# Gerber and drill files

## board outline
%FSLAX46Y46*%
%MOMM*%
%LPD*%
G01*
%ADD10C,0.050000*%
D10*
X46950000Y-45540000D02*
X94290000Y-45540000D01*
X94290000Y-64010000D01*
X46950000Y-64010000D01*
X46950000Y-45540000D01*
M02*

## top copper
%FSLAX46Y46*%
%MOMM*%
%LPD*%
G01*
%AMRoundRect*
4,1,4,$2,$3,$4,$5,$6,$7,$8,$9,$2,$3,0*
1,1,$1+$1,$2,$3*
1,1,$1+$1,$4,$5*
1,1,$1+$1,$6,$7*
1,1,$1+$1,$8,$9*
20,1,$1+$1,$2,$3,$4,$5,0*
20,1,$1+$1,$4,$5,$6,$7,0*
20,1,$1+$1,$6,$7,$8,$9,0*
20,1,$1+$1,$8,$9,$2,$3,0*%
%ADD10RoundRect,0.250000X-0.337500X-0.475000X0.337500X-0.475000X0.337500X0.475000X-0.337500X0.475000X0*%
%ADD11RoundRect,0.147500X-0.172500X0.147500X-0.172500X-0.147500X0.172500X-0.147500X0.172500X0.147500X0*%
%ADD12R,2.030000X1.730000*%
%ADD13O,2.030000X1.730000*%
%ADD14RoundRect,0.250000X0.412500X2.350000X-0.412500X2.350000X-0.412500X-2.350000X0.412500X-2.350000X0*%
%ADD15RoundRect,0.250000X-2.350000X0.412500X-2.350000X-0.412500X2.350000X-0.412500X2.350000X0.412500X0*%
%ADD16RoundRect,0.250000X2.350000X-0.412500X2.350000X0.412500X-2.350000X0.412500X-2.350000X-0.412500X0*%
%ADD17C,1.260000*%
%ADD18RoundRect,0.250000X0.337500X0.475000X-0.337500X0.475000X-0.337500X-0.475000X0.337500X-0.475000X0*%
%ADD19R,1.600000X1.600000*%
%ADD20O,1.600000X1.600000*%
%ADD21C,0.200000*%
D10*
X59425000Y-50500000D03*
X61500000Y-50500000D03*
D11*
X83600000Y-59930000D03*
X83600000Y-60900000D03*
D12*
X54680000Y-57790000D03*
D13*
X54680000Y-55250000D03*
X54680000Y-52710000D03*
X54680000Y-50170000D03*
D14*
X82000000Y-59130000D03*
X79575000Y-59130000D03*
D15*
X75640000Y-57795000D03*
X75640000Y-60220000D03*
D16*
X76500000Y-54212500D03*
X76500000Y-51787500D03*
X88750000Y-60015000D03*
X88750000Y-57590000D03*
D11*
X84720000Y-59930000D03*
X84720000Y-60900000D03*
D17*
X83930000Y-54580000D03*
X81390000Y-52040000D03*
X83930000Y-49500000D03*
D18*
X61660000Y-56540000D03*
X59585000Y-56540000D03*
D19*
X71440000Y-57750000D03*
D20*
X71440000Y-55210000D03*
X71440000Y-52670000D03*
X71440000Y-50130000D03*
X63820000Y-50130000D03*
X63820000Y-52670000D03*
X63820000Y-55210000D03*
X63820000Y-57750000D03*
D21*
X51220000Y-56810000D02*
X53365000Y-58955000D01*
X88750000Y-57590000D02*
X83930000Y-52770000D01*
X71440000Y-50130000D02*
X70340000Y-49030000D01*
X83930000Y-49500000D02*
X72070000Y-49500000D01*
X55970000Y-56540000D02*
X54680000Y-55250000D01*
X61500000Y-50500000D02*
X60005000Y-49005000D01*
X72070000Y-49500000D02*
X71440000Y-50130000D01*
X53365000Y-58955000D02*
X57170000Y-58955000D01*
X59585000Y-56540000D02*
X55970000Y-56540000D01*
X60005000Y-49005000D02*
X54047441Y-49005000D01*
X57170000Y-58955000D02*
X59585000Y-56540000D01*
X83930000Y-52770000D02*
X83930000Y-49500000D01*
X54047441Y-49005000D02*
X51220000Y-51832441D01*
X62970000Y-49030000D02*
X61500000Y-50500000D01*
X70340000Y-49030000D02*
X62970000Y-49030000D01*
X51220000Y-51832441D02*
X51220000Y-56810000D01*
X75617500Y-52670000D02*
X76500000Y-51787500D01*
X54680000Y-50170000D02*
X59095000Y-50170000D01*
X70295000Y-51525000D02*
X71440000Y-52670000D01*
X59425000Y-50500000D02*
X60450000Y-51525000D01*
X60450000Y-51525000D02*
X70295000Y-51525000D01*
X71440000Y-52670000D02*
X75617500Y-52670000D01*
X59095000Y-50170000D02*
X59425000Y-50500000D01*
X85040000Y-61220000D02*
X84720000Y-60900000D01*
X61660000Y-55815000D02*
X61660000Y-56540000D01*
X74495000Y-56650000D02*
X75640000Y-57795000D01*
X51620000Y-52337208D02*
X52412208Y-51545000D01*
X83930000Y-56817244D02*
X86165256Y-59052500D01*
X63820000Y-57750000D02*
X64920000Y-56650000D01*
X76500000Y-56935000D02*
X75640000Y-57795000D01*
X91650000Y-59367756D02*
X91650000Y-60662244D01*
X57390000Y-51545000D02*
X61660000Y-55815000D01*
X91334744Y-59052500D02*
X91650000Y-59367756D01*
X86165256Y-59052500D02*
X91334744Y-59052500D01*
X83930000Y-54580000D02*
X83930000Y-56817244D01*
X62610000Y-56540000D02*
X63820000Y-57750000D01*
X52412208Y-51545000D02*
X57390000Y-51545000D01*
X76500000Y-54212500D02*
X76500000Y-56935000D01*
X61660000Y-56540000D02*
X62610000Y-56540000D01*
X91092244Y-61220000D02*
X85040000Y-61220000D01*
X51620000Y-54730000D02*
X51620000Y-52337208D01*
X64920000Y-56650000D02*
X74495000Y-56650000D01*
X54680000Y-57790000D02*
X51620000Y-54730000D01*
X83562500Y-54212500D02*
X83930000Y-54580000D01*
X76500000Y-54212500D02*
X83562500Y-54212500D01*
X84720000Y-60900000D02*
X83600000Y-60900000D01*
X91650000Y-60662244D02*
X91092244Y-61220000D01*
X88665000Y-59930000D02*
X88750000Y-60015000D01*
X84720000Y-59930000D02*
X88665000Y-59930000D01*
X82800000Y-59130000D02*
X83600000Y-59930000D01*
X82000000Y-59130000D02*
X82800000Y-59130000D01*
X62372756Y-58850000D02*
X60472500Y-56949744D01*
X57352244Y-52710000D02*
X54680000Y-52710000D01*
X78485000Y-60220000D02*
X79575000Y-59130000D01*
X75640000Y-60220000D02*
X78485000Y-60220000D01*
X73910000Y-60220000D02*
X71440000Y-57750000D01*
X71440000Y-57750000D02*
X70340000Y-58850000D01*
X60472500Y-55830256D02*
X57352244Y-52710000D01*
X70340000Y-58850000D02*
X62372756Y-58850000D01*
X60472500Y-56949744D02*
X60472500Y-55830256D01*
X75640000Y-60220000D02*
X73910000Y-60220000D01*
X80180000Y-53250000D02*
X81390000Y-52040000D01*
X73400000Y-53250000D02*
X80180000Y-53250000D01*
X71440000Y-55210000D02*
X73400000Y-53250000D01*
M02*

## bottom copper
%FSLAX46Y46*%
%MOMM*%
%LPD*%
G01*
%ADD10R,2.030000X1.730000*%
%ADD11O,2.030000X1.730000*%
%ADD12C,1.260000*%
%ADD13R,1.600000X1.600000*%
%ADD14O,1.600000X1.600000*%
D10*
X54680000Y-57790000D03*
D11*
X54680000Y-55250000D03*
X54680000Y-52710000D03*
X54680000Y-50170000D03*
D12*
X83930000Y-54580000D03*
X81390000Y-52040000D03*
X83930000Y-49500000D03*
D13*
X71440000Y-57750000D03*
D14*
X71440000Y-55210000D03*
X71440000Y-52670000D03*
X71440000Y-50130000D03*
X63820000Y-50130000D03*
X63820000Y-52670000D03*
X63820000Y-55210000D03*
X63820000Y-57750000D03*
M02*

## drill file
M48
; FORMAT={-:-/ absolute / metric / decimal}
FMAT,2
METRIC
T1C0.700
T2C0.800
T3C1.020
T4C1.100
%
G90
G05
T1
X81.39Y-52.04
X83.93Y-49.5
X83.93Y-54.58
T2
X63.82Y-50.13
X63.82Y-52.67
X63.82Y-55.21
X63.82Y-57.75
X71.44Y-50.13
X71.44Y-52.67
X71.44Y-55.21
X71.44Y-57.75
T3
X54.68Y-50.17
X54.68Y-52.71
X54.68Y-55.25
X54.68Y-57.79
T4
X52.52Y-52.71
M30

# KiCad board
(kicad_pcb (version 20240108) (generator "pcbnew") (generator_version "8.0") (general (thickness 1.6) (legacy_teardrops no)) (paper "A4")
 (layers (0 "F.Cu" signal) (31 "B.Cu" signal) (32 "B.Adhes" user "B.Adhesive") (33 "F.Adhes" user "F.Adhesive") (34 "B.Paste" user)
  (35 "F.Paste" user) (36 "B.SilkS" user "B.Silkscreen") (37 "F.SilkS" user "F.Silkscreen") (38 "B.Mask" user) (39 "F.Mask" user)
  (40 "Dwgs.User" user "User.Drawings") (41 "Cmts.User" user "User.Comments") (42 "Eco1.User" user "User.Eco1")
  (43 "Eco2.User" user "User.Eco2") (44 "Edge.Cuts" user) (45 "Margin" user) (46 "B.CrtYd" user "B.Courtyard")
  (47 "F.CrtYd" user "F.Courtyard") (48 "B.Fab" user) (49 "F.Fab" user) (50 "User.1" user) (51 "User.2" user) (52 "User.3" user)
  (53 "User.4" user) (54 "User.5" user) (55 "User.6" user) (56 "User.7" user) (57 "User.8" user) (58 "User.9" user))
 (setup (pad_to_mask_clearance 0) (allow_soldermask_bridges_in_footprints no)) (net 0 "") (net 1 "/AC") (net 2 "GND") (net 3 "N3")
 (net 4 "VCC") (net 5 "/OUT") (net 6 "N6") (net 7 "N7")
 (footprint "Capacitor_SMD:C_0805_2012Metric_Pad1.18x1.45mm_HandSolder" (layer "F.Cu") (at 60.4625 50.5)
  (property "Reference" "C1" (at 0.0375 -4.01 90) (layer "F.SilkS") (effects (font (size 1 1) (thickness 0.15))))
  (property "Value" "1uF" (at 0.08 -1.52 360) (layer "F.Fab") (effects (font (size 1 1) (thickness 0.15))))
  (pad "1" smd roundrect (at -1.0375 0) (size 1.175 1.45) (layers "F.Cu" "F.Paste" "F.Mask") (roundrect_rratio 0.212766) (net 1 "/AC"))
  (pad "2" smd roundrect (at 1.0375 0) (size 1.175 1.45) (layers "F.Cu" "F.Paste" "F.Mask") (roundrect_rratio 0.212766) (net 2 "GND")))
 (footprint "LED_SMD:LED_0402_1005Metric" (layer "F.Cu") (at 83.6 60.415 -90)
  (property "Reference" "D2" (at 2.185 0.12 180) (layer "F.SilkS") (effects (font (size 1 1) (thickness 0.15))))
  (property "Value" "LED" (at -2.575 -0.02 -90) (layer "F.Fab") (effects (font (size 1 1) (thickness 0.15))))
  (pad "1" smd roundrect (at -0.485 0 270) (size 0.59 0.64) (layers "F.Cu" "F.Paste" "F.Mask") (roundrect_rratio 0.25) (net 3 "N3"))
  (pad "2" smd roundrect (at 0.485 0 270) (size 0.59 0.64) (layers "F.Cu" "F.Paste" "F.Mask") (roundrect_rratio 0.25) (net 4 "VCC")))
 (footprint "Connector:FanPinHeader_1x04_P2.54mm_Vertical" (layer "F.Cu") (at 54.68 57.79 90)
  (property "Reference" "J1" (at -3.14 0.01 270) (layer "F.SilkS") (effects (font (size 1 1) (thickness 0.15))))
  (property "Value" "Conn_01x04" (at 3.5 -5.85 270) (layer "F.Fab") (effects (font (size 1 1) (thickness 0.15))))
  (pad "" np_thru_hole circle (at 5.08 -2.16 180) (size 1.1 1.1) (drill 1.1) (layers "*.Cu" "*.Mask"))
  (pad "1" thru_hole rect (at 0 0 180) (size 2.03 1.73) (drill 1.02) (layers "*.Cu" "*.Mask") (remove_unused_layers no) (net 4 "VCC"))
  (pad "2" thru_hole oval (at 2.54 0 180) (size 2.03 1.73) (drill 1.02) (layers "*.Cu" "*.Mask") (remove_unused_layers no) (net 2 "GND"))
  (pad "3" thru_hole oval (at 5.08 0 180) (size 2.03 1.73) (drill 1.02) (layers "*.Cu" "*.Mask") (remove_unused_layers no) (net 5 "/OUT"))
  (pad "4" thru_hole oval (at 7.62 0 180) (size 2.03 1.73) (drill 1.02) (layers "*.Cu" "*.Mask") (remove_unused_layers no) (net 1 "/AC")))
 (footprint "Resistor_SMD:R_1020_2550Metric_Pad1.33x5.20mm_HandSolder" (layer "F.Cu") (at 80.7875 59.13 180)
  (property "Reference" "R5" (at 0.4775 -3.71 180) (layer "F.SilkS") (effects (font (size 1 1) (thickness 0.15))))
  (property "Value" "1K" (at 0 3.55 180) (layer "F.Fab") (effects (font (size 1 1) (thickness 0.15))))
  (pad "1" smd roundrect (at -1.2125 0 180) (size 1.325 5.2) (layers "F.Cu" "F.Paste" "F.Mask") (roundrect_rratio 0.188679) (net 3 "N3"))
  (pad "2" smd roundrect (at 1.2125 0 180) (size 1.325 5.2) (layers "F.Cu" "F.Paste" "F.Mask") (roundrect_rratio 0.188679) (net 5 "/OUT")))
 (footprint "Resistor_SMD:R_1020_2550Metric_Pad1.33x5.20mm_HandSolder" (layer "F.Cu") (at 75.64 59.0075 -90)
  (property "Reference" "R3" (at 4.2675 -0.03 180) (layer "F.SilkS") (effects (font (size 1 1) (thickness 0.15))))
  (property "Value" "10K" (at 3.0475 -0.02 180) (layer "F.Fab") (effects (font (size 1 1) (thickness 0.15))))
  (pad "1" smd roundrect (at -1.2125 0 270) (size 1.325 5.2) (layers "F.Cu" "F.Paste" "F.Mask") (roundrect_rratio 0.188679) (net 4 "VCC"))
  (pad "2" smd roundrect (at 1.2125 0 270) (size 1.325 5.2) (layers "F.Cu" "F.Paste" "F.Mask") (roundrect_rratio 0.188679) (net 5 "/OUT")))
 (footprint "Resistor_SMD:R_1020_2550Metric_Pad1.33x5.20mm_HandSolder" (layer "F.Cu") (at 76.5 53 90)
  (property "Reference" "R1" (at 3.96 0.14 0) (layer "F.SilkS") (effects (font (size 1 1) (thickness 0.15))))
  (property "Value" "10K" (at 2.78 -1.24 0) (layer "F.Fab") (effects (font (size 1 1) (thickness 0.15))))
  (pad "1" smd roundrect (at -1.2125 0 90) (size 1.325 5.2) (layers "F.Cu" "F.Paste" "F.Mask") (roundrect_rratio 0.188679) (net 4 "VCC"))
  (pad "2" smd roundrect (at 1.2125 0 90) (size 1.325 5.2) (layers "F.Cu" "F.Paste" "F.Mask") (roundrect_rratio 0.188679) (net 1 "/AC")))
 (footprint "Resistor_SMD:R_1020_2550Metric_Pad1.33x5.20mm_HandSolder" (layer "F.Cu") (at 88.75 58.8025 90)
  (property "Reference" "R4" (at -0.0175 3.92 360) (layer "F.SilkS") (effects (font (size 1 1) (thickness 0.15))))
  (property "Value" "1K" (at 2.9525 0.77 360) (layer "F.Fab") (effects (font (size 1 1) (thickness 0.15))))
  (pad "1" smd roundrect (at -1.2125 0 90) (size 1.325 5.2) (layers "F.Cu" "F.Paste" "F.Mask") (roundrect_rratio 0.188679) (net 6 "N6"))
  (pad "2" smd roundrect (at 1.2125 0 90) (size 1.325 5.2) (layers "F.Cu" "F.Paste" "F.Mask") (roundrect_rratio 0.188679) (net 2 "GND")))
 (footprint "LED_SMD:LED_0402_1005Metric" (layer "F.Cu") (at 84.72 60.415 -90)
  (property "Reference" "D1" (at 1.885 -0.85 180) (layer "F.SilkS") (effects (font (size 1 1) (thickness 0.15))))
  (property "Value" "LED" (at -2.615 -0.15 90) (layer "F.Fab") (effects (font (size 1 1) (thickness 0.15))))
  (pad "1" smd roundrect (at -0.485 0 270) (size 0.59 0.64) (layers "F.Cu" "F.Paste" "F.Mask") (roundrect_rratio 0.25) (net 6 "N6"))
  (pad "2" smd roundrect (at 0.485 0 270) (size 0.59 0.64) (layers "F.Cu" "F.Paste" "F.Mask") (roundrect_rratio 0.25) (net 4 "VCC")))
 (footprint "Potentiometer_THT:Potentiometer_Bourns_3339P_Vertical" (layer "F.Cu") (at 83.93 54.58)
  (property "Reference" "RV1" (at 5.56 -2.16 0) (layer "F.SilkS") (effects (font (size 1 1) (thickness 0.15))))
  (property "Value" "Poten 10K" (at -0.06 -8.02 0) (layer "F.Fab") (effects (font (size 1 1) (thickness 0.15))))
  (pad "1" thru_hole circle (at 0 0) (size 1.26 1.26) (drill 0.7) (layers "*.Cu" "*.Mask") (remove_unused_layers no) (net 4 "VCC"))
  (pad "2" thru_hole circle (at -2.54 -2.54) (size 1.26 1.26) (drill 0.7) (layers "*.Cu" "*.Mask") (remove_unused_layers no) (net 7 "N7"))
  (pad "3" thru_hole circle (at 0 -5.08) (size 1.26 1.26) (drill 0.7) (layers "*.Cu" "*.Mask") (remove_unused_layers no) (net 2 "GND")))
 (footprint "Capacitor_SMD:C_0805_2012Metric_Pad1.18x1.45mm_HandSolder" (layer "F.Cu") (at 60.6225 56.54 180)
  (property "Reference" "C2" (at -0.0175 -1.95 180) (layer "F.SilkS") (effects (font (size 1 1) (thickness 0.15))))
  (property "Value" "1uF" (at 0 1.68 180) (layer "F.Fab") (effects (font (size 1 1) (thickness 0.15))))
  (pad "1" smd roundrect (at -1.0375 0 180) (size 1.175 1.45) (layers "F.Cu" "F.Paste" "F.Mask") (roundrect_rratio 0.212766) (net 4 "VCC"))
  (pad "2" smd roundrect (at 1.0375 0 180) (size 1.175 1.45) (layers "F.Cu" "F.Paste" "F.Mask") (roundrect_rratio 0.212766) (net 2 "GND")))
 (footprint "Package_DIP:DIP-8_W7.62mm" (layer "F.Cu") (at 71.44 57.75 180)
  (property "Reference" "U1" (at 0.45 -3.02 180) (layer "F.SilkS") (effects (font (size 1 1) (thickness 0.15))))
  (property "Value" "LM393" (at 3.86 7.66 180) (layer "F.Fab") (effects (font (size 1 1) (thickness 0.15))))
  (pad "1" thru_hole rect (at 0 0 180) (size 1.6 1.6) (drill 0.8) (layers "*.Cu" "*.Mask") (remove_unused_layers no) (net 5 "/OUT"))
  (pad "2" thru_hole oval (at 0 2.54 180) (size 1.6 1.6) (drill 0.8) (layers "*.Cu" "*.Mask") (remove_unused_layers no) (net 7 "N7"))
  (pad "3" thru_hole oval (at 0 5.08 180) (size 1.6 1.6) (drill 0.8) (layers "*.Cu" "*.Mask") (remove_unused_layers no) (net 1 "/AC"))
  (pad "4" thru_hole oval (at 0 7.62 180) (size 1.6 1.6) (drill 0.8) (layers "*.Cu" "*.Mask") (remove_unused_layers no) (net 2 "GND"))
  (pad "5" thru_hole oval (at 7.62 7.62 180) (size 1.6 1.6) (drill 0.8) (layers "*.Cu" "*.Mask") (remove_unused_layers no))
  (pad "6" thru_hole oval (at 7.62 5.08 180) (size 1.6 1.6) (drill 0.8) (layers "*.Cu" "*.Mask") (remove_unused_layers no))
  (pad "7" thru_hole oval (at 7.62 2.54 180) (size 1.6 1.6) (drill 0.8) (layers "*.Cu" "*.Mask") (remove_unused_layers no))
  (pad "8" thru_hole oval (at 7.62 0 180) (size 1.6 1.6) (drill 0.8) (layers "*.Cu" "*.Mask") (remove_unused_layers no) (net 4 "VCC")))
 (gr_rect (start 46.95 45.54) (end 94.29 64.01) (stroke (width 0.05) (type default)) (fill none) (layer "Edge.Cuts"))
 (segment (start 51.22 56.81) (end 53.365 58.955) (width 0.2) (layer "F.Cu") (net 2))
 (segment (start 88.75 57.59) (end 83.93 52.77) (width 0.2) (layer "F.Cu") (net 2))
 (segment (start 71.44 50.13) (end 70.34 49.03) (width 0.2) (layer "F.Cu") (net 2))
 (segment (start 83.93 49.5) (end 72.07 49.5) (width 0.2) (layer "F.Cu") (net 2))
 (segment (start 55.97 56.54) (end 54.68 55.25) (width 0.2) (layer "F.Cu") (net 2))
 (segment (start 61.5 50.5) (end 60.005 49.005) (width 0.2) (layer "F.Cu") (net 2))
 (segment (start 72.07 49.5) (end 71.44 50.13) (width 0.2) (layer "F.Cu") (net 2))
 (segment (start 53.365 58.955) (end 57.17 58.955) (width 0.2) (layer "F.Cu") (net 2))
 (segment (start 59.585 56.54) (end 55.97 56.54) (width 0.2) (layer "F.Cu") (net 2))
 (segment (start 60.005 49.005) (end 54.047441 49.005) (width 0.2) (layer "F.Cu") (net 2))
 (segment (start 57.17 58.955) (end 59.585 56.54) (width 0.2) (layer "F.Cu") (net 2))
 (segment (start 83.93 52.77) (end 83.93 49.5) (width 0.2) (layer "F.Cu") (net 2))
 (segment (start 54.047441 49.005) (end 51.22 51.832441) (width 0.2) (layer "F.Cu") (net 2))
 (segment (start 62.97 49.03) (end 61.5 50.5) (width 0.2) (layer "F.Cu") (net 2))
 (segment (start 70.34 49.03) (end 62.97 49.03) (width 0.2) (layer "F.Cu") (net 2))
 (segment (start 51.22 51.832441) (end 51.22 56.81) (width 0.2) (layer "F.Cu") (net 2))
 (segment (start 75.6175 52.67) (end 76.5 51.7875) (width 0.2) (layer "F.Cu") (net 1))
 (segment (start 54.68 50.17) (end 59.095 50.17) (width 0.2) (layer "F.Cu") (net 1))
 (segment (start 70.295 51.525) (end 71.44 52.67) (width 0.2) (layer "F.Cu") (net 1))
 (segment (start 59.425 50.5) (end 60.45 51.525) (width 0.2) (layer "F.Cu") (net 1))
 (segment (start 60.45 51.525) (end 70.295 51.525) (width 0.2) (layer "F.Cu") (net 1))
 (segment (start 71.44 52.67) (end 75.6175 52.67) (width 0.2) (layer "F.Cu") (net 1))
 (segment (start 59.095 50.17) (end 59.425 50.5) (width 0.2) (layer "F.Cu") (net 1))
 (segment (start 85.04 61.22) (end 84.72 60.9) (width 0.2) (layer "F.Cu") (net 4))
 (segment (start 61.66 55.815) (end 61.66 56.54) (width 0.2) (layer "F.Cu") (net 4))
 (segment (start 74.495 56.65) (end 75.64 57.795) (width 0.2) (layer "F.Cu") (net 4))
 (segment (start 51.62 52.337208) (end 52.412208 51.545) (width 0.2) (layer "F.Cu") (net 4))
 (segment (start 83.93 56.817244) (end 86.165256 59.0525) (width 0.2) (layer "F.Cu") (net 4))
 (segment (start 63.82 57.75) (end 64.92 56.65) (width 0.2) (layer "F.Cu") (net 4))
 (segment (start 76.5 56.935) (end 75.64 57.795) (width 0.2) (layer "F.Cu") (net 4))
 (segment (start 91.65 59.367756) (end 91.65 60.662244) (width 0.2) (layer "F.Cu") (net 4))
 (segment (start 57.39 51.545) (end 61.66 55.815) (width 0.2) (layer "F.Cu") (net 4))
 (segment (start 91.334744 59.0525) (end 91.65 59.367756) (width 0.2) (layer "F.Cu") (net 4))
 (segment (start 86.165256 59.0525) (end 91.334744 59.0525) (width 0.2) (layer "F.Cu") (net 4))
 (segment (start 83.93 54.58) (end 83.93 56.817244) (width 0.2) (layer "F.Cu") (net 4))
 (segment (start 62.61 56.54) (end 63.82 57.75) (width 0.2) (layer "F.Cu") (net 4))
 (segment (start 52.412208 51.545) (end 57.39 51.545) (width 0.2) (layer "F.Cu") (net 4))
 (segment (start 76.5 54.2125) (end 76.5 56.935) (width 0.2) (layer "F.Cu") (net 4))
 (segment (start 61.66 56.54) (end 62.61 56.54) (width 0.2) (layer "F.Cu") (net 4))
 (segment (start 91.092244 61.22) (end 85.04 61.22) (width 0.2) (layer "F.Cu") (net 4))
 (segment (start 51.62 54.73) (end 51.62 52.337208) (width 0.2) (layer "F.Cu") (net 4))
 (segment (start 64.92 56.65) (end 74.495 56.65) (width 0.2) (layer "F.Cu") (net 4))
 (segment (start 54.68 57.79) (end 51.62 54.73) (width 0.2) (layer "F.Cu") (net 4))
 (segment (start 83.5625 54.2125) (end 83.93 54.58) (width 0.2) (layer "F.Cu") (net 4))
 (segment (start 76.5 54.2125) (end 83.5625 54.2125) (width 0.2) (layer "F.Cu") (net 4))
 (segment (start 84.72 60.9) (end 83.6 60.9) (width 0.2) (layer "F.Cu") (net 4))
 (segment (start 91.65 60.662244) (end 91.092244 61.22) (width 0.2) (layer "F.Cu") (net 4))
 (segment (start 88.665 59.93) (end 88.75 60.015) (width 0.2) (layer "F.Cu") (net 6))
 (segment (start 84.72 59.93) (end 88.665 59.93) (width 0.2) (layer "F.Cu") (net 6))
 (segment (start 82.8 59.13) (end 83.6 59.93) (width 0.2) (layer "F.Cu") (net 3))
 (segment (start 82 59.13) (end 82.8 59.13) (width 0.2) (layer "F.Cu") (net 3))
 (segment (start 62.372756 58.85) (end 60.4725 56.949744) (width 0.2) (layer "F.Cu") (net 5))
 (segment (start 57.352244 52.71) (end 54.68 52.71) (width 0.2) (layer "F.Cu") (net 5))
 (segment (start 78.485 60.22) (end 79.575 59.13) (width 0.2) (layer "F.Cu") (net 5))
 (segment (start 75.64 60.22) (end 78.485 60.22) (width 0.2) (layer "F.Cu") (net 5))
 (segment (start 73.91 60.22) (end 71.44 57.75) (width 0.2) (layer "F.Cu") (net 5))
 (segment (start 71.44 57.75) (end 70.34 58.85) (width 0.2) (layer "F.Cu") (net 5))
 (segment (start 60.4725 55.830256) (end 57.352244 52.71) (width 0.2) (layer "F.Cu") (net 5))
 (segment (start 70.34 58.85) (end 62.372756 58.85) (width 0.2) (layer "F.Cu") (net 5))
 (segment (start 60.4725 56.949744) (end 60.4725 55.830256) (width 0.2) (layer "F.Cu") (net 5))
 (segment (start 75.64 60.22) (end 73.91 60.22) (width 0.2) (layer "F.Cu") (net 5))
 (segment (start 80.18 53.25) (end 81.39 52.04) (width 0.2) (layer "F.Cu") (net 7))
 (segment (start 73.4 53.25) (end 80.18 53.25) (width 0.2) (layer "F.Cu") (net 7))
 (segment (start 71.44 55.21) (end 73.4 53.25) (width 0.2) (layer "F.Cu") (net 7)))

